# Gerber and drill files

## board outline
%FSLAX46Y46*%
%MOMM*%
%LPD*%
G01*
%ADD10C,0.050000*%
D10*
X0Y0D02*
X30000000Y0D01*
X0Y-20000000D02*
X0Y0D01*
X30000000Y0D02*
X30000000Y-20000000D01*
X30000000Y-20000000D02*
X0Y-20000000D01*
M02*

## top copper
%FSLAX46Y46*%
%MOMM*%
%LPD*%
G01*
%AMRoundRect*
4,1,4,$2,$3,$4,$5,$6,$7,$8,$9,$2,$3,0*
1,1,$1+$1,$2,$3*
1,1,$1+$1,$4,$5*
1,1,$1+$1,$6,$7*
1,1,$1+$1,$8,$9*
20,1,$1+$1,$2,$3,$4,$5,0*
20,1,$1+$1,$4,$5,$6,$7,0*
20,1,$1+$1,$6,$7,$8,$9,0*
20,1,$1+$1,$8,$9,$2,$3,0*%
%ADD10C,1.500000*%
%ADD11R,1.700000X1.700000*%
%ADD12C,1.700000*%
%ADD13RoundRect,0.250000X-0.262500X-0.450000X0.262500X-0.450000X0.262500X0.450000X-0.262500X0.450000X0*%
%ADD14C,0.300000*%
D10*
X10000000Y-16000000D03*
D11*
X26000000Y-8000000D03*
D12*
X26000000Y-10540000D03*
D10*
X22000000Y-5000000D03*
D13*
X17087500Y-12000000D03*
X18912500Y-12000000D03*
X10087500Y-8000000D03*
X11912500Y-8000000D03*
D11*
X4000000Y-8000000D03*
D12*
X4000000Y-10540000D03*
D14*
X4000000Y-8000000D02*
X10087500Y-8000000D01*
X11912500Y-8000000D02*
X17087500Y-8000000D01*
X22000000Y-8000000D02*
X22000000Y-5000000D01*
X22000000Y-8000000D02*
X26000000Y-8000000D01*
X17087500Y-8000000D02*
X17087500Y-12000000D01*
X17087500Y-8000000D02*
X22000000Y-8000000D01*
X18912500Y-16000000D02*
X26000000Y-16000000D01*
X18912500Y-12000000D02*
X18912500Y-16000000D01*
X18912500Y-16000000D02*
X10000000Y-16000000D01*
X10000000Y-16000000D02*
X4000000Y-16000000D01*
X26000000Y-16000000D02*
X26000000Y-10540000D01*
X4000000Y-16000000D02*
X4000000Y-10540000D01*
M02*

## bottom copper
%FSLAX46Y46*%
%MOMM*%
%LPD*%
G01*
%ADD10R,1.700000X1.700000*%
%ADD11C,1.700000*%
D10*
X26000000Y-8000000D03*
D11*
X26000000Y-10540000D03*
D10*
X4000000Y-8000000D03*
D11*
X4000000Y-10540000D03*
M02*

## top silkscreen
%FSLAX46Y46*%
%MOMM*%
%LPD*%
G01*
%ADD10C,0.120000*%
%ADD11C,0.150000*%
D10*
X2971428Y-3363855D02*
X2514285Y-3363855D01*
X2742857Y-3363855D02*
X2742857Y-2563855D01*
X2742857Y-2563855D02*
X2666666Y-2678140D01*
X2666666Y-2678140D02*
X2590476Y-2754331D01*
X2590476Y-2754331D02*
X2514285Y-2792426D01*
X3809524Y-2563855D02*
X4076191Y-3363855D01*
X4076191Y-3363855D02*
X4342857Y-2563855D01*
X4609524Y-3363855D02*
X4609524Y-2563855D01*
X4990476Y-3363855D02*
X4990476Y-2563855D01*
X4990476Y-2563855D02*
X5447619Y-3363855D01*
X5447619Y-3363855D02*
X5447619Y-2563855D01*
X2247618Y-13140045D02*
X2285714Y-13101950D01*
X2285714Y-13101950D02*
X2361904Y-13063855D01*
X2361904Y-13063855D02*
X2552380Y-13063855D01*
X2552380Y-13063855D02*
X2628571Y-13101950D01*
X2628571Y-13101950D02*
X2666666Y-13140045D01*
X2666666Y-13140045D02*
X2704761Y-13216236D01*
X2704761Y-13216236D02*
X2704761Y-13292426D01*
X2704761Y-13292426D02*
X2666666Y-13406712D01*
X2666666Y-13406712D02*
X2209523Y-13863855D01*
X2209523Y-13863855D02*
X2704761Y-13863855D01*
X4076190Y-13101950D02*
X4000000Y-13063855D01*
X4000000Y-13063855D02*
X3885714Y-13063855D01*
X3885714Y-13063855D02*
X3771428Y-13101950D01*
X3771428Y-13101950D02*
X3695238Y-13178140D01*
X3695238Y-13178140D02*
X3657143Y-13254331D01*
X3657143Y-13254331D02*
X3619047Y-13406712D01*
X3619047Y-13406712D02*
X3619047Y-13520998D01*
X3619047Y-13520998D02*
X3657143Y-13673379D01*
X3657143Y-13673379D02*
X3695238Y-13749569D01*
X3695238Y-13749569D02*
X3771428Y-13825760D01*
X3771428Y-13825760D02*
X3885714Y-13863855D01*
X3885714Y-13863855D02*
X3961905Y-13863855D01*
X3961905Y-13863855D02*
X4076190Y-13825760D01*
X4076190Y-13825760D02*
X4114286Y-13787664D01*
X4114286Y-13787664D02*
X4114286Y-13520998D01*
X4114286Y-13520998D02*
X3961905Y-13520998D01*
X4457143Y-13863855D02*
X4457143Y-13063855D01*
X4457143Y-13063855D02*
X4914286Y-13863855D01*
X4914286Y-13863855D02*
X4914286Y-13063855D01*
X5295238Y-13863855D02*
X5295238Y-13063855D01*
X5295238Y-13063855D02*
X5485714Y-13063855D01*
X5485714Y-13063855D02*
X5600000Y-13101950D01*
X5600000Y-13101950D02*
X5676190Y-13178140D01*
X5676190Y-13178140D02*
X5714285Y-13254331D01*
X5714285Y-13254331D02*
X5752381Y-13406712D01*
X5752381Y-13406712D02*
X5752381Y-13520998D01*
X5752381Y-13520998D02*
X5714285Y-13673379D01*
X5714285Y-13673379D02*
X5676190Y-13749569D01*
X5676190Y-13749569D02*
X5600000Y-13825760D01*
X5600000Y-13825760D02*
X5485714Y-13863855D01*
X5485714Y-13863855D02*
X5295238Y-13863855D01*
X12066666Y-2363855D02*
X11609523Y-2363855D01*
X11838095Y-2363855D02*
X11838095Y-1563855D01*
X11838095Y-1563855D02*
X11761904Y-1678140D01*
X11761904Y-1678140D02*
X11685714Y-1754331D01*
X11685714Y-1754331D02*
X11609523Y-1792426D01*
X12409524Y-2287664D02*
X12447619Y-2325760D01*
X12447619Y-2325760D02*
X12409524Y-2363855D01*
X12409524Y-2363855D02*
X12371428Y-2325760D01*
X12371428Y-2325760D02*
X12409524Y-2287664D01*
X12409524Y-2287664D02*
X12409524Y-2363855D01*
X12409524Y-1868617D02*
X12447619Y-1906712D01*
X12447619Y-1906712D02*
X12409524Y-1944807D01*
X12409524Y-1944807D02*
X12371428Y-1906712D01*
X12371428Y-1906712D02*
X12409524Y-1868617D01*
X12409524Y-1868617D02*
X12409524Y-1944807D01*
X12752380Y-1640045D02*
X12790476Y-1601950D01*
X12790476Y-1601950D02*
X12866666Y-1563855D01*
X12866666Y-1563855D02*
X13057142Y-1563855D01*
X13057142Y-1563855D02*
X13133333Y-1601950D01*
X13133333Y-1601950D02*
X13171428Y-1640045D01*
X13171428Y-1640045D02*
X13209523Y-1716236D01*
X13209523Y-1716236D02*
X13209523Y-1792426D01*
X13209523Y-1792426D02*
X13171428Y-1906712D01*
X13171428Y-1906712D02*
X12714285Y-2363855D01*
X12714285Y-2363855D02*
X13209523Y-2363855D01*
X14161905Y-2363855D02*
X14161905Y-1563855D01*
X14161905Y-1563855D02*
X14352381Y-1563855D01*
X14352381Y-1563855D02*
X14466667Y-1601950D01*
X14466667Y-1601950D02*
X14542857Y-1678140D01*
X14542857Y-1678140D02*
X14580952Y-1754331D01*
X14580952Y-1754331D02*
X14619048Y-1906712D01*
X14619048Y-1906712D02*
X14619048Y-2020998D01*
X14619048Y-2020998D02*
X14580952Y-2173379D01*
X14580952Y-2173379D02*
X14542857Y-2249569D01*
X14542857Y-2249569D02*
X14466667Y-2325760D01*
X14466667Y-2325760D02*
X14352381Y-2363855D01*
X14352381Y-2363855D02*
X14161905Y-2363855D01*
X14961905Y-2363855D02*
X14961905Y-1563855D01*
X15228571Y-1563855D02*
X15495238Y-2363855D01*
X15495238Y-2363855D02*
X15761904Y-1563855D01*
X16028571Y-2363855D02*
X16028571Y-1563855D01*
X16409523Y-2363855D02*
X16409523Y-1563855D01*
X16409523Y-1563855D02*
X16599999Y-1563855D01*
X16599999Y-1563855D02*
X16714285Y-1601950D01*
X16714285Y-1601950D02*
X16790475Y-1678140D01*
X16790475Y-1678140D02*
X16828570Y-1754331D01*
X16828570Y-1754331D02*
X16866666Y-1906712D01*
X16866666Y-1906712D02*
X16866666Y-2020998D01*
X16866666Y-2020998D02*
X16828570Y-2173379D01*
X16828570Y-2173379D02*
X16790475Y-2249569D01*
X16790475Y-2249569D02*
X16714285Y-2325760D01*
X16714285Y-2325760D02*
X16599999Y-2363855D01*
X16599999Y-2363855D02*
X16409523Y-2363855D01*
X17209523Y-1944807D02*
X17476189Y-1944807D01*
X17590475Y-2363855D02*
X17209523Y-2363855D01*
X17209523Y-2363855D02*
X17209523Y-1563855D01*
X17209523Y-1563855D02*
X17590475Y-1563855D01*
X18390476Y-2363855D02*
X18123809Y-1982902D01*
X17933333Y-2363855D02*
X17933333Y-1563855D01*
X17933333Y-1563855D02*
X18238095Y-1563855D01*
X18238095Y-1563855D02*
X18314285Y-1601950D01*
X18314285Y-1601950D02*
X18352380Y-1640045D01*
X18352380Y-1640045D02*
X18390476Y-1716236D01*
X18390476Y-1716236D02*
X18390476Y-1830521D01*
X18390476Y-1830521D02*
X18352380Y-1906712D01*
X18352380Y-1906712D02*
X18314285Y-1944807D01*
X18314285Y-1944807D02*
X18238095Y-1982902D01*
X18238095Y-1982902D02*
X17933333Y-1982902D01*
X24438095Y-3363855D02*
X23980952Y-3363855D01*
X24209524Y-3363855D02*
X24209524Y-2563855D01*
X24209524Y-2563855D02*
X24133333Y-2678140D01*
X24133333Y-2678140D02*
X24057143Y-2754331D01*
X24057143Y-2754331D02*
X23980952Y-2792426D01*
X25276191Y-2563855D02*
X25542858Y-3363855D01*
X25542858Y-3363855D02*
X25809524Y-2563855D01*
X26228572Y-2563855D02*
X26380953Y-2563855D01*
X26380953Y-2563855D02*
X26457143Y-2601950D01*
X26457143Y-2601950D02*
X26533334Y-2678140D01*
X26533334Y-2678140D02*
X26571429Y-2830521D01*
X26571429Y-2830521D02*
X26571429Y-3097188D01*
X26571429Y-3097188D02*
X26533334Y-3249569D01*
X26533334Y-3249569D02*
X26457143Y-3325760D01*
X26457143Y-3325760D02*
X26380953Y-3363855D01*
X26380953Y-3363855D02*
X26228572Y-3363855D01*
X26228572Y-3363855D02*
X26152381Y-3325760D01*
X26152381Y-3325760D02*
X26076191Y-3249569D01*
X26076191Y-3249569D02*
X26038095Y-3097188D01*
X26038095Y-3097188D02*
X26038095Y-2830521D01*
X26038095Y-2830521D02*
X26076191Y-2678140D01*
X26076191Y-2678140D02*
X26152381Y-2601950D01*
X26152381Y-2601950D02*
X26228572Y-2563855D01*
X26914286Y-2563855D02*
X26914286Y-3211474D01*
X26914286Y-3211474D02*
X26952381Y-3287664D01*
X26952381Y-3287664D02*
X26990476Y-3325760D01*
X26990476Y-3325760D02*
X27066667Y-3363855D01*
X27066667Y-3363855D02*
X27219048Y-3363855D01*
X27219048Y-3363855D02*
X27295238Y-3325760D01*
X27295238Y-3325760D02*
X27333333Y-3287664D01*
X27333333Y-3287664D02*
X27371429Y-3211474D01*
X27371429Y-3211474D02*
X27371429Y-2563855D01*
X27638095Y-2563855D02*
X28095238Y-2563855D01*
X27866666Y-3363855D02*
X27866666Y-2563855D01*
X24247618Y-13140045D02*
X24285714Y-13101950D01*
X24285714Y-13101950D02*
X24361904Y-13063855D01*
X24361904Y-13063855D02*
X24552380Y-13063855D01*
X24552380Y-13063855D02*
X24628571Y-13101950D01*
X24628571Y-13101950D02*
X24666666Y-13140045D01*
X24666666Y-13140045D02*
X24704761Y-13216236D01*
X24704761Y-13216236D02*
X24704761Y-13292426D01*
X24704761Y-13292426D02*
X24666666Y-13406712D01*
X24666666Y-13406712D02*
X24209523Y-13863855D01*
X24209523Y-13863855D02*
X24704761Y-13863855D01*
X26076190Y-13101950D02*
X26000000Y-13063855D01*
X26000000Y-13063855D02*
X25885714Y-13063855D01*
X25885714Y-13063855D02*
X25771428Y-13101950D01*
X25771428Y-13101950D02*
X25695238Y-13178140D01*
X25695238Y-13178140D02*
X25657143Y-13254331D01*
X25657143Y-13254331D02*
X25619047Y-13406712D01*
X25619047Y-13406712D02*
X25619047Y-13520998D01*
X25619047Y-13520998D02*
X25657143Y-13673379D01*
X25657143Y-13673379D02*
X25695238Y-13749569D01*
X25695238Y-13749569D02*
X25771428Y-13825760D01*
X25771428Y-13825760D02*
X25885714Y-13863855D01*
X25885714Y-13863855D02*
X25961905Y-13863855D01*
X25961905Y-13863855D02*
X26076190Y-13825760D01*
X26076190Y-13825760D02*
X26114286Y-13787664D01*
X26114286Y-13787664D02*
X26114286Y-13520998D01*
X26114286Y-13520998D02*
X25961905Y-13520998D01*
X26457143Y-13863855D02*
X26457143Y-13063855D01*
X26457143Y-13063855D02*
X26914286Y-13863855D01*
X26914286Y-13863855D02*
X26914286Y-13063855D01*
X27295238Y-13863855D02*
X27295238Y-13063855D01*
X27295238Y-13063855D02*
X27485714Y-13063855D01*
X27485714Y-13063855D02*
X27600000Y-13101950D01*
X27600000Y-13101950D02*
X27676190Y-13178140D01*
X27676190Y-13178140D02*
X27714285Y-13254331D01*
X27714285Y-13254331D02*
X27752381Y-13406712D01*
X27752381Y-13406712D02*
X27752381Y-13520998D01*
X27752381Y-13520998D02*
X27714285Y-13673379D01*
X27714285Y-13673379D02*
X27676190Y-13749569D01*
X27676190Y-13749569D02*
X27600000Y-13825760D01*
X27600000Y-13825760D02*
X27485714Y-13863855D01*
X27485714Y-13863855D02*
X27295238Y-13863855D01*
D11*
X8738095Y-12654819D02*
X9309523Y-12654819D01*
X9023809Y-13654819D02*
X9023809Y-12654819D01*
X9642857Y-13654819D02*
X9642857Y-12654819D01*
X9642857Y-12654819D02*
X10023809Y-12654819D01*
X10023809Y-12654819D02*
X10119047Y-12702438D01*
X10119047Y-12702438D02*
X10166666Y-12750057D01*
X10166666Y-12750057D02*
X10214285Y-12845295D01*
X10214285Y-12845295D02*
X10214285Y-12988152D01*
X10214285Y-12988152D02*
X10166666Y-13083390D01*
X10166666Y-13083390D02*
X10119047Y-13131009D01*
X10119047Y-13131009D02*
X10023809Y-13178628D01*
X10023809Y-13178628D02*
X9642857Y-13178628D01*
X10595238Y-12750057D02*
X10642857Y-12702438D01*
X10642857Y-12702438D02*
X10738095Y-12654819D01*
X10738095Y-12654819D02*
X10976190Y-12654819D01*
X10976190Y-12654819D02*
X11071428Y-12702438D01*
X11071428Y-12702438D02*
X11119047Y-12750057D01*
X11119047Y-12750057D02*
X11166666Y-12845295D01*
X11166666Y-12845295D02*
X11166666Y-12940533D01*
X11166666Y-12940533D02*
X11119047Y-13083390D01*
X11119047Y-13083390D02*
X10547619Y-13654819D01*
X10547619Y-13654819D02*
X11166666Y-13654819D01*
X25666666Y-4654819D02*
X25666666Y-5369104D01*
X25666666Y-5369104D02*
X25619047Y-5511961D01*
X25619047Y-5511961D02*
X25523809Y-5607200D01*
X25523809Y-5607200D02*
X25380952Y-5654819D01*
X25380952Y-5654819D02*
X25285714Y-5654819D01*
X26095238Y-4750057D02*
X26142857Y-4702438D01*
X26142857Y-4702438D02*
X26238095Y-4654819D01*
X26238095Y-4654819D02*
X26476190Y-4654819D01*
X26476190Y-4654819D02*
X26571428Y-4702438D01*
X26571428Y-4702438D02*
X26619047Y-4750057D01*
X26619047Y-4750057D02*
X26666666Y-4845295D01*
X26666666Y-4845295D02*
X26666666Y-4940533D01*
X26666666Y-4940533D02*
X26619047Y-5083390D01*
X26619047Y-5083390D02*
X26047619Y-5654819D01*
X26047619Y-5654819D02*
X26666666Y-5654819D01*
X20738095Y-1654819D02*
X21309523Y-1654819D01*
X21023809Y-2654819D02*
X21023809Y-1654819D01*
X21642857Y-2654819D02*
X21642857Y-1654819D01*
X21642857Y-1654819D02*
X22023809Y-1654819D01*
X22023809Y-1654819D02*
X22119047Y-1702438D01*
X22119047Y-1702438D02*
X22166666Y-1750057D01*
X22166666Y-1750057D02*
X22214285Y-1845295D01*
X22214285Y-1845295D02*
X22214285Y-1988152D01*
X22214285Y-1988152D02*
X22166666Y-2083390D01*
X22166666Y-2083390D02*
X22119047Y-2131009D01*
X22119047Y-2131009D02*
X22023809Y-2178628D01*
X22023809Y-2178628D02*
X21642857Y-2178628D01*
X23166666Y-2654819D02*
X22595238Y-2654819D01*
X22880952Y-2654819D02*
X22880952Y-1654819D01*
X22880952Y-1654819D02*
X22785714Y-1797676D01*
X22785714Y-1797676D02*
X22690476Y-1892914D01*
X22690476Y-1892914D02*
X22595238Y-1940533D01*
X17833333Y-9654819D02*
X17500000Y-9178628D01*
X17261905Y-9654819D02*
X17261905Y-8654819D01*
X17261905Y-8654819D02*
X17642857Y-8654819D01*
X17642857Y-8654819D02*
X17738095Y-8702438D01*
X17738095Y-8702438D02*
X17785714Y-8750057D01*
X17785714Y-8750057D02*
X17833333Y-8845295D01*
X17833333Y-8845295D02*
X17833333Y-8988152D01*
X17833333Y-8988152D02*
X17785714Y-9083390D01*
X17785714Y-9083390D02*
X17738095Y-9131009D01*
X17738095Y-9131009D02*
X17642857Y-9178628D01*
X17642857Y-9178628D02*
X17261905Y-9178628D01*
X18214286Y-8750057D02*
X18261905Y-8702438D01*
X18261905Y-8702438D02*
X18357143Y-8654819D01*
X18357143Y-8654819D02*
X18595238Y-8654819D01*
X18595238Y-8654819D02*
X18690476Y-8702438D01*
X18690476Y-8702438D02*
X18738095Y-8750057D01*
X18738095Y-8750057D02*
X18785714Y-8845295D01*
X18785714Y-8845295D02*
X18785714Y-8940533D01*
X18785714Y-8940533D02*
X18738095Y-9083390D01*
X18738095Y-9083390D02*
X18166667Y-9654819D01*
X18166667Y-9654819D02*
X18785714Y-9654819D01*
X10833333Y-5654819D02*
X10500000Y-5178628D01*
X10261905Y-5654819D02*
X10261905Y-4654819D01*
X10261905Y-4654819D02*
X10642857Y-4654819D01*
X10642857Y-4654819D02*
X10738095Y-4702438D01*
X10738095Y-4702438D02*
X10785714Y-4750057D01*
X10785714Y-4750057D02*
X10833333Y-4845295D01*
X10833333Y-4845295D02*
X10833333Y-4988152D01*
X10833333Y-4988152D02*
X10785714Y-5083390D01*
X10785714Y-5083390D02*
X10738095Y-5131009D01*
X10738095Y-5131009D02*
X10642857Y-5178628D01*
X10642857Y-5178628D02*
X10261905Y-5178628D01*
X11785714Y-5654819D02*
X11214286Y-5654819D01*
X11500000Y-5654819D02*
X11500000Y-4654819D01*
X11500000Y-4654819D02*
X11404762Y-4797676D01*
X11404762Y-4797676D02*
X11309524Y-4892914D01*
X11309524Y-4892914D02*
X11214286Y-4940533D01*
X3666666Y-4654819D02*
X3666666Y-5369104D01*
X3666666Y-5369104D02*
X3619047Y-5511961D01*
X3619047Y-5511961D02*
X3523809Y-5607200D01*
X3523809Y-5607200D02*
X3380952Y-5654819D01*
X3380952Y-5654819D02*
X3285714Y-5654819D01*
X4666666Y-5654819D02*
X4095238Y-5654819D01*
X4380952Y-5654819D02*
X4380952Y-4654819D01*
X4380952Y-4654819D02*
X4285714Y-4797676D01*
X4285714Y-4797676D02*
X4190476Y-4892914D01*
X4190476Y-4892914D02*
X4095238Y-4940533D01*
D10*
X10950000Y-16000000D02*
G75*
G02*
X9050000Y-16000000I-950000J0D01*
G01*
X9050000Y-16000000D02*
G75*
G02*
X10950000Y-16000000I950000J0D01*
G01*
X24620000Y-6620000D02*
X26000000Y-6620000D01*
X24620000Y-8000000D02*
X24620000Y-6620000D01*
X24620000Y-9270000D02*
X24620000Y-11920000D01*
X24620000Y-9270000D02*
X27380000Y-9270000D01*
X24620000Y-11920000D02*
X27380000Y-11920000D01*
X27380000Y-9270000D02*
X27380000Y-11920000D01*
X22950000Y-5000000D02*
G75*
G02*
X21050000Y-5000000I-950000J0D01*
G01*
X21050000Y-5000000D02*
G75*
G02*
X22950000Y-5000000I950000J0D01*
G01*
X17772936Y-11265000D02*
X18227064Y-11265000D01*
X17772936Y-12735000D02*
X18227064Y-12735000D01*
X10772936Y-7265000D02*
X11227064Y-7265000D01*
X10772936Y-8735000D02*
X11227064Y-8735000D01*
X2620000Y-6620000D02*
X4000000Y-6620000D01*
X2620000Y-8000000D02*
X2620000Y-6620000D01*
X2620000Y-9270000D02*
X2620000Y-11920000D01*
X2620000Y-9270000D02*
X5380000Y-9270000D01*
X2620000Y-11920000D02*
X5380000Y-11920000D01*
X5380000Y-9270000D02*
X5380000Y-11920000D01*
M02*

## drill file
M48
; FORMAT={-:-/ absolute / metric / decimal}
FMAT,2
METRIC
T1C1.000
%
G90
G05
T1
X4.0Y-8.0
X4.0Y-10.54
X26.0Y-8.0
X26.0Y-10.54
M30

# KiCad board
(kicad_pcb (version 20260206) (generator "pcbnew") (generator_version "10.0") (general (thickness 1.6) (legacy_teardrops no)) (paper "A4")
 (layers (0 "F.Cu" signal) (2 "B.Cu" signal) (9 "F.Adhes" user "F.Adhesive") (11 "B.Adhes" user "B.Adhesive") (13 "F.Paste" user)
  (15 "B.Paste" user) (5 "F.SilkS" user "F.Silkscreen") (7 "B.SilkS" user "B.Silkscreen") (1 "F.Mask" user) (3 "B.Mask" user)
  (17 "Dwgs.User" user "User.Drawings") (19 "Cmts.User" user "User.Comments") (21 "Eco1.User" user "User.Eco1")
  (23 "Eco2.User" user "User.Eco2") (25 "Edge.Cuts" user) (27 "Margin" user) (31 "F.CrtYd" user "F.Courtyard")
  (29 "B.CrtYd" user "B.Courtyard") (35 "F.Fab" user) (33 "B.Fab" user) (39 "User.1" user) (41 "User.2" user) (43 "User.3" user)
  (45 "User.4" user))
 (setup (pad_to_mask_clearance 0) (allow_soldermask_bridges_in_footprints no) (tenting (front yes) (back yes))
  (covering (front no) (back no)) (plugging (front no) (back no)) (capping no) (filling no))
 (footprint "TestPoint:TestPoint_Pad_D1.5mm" (layer "F.Cu") (at 10 16)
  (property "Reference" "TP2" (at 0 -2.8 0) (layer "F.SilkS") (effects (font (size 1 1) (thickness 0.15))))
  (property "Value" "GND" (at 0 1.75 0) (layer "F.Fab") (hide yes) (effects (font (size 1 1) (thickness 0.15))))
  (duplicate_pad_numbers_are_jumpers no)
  (fp_circle (center 0 0) (end 0 0.95) (stroke (width 0.12) (type solid)) (fill no) (layer "F.SilkS"))
  (pad "1" smd circle (at 0 0) (size 1.5 1.5) (layers "F.Cu" "F.Mask") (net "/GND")))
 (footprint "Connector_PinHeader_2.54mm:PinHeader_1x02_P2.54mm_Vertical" (layer "F.Cu") (at 26 8)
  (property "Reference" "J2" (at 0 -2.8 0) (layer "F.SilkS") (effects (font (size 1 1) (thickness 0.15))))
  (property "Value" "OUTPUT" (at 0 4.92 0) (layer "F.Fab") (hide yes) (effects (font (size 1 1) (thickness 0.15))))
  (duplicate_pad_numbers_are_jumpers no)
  (fp_line (start -1.38 -1.38) (end 0 -1.38) (stroke (width 0.12) (type solid)) (layer "F.SilkS"))
  (fp_line (start -1.38 0) (end -1.38 -1.38) (stroke (width 0.12) (type solid)) (layer "F.SilkS"))
  (fp_line (start -1.38 1.27) (end -1.38 3.92) (stroke (width 0.12) (type solid)) (layer "F.SilkS"))
  (fp_line (start -1.38 1.27) (end 1.38 1.27) (stroke (width 0.12) (type solid)) (layer "F.SilkS"))
  (fp_line (start -1.38 3.92) (end 1.38 3.92) (stroke (width 0.12) (type solid)) (layer "F.SilkS"))
  (fp_line (start 1.38 1.27) (end 1.38 3.92) (stroke (width 0.12) (type solid)) (layer "F.SilkS"))
  (pad "1" thru_hole rect (at 0 0) (size 1.7 1.7) (drill 1) (layers "*.Cu" "*.Mask") (remove_unused_layers no) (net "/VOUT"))
  (pad "2" thru_hole circle (at 0 2.54) (size 1.7 1.7) (drill 1) (layers "*.Cu" "*.Mask") (remove_unused_layers no) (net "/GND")))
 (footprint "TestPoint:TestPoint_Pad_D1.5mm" (layer "F.Cu") (at 22 5)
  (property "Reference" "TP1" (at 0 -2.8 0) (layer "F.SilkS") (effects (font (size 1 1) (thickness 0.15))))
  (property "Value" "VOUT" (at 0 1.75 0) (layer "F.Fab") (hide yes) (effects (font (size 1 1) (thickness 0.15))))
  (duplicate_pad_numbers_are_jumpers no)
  (fp_circle (center 0 0) (end 0 0.95) (stroke (width 0.12) (type solid)) (fill no) (layer "F.SilkS"))
  (pad "1" smd circle (at 0 0) (size 1.5 1.5) (layers "F.Cu" "F.Mask") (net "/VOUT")))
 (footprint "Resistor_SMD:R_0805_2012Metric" (layer "F.Cu") (at 18 12)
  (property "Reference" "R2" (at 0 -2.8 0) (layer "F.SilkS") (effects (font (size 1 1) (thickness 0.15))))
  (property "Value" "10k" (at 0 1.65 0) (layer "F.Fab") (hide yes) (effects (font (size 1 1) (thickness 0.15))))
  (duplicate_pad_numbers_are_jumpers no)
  (fp_line (start -0.227064 -0.735) (end 0.227064 -0.735) (stroke (width 0.12) (type solid)) (layer "F.SilkS"))
  (fp_line (start -0.227064 0.735) (end 0.227064 0.735) (stroke (width 0.12) (type solid)) (layer "F.SilkS"))
  (pad "1" smd roundrect (at -0.9125 0) (size 1.025 1.4) (layers "F.Cu" "F.Mask" "F.Paste") (roundrect_rratio 0.243902) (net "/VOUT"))
  (pad "2" smd roundrect (at 0.9125 0) (size 1.025 1.4) (layers "F.Cu" "F.Mask" "F.Paste") (roundrect_rratio 0.243902) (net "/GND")))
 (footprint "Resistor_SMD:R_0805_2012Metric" (layer "F.Cu") (at 11 8)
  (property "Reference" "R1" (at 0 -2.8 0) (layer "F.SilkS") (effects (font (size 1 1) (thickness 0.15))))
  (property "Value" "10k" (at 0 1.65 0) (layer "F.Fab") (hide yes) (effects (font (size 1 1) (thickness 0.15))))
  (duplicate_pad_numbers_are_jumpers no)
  (fp_line (start -0.227064 -0.735) (end 0.227064 -0.735) (stroke (width 0.12) (type solid)) (layer "F.SilkS"))
  (fp_line (start -0.227064 0.735) (end 0.227064 0.735) (stroke (width 0.12) (type solid)) (layer "F.SilkS"))
  (pad "1" smd roundrect (at -0.9125 0) (size 1.025 1.4) (layers "F.Cu" "F.Mask" "F.Paste") (roundrect_rratio 0.243902) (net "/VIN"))
  (pad "2" smd roundrect (at 0.9125 0) (size 1.025 1.4) (layers "F.Cu" "F.Mask" "F.Paste") (roundrect_rratio 0.243902) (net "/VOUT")))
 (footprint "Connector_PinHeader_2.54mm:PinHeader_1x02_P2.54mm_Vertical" (layer "F.Cu") (at 4 8)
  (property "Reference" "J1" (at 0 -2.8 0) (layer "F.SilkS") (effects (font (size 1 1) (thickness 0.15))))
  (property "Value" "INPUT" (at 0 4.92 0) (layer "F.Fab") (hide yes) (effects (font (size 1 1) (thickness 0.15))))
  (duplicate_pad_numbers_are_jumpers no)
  (fp_line (start -1.38 -1.38) (end 0 -1.38) (stroke (width 0.12) (type solid)) (layer "F.SilkS"))
  (fp_line (start -1.38 0) (end -1.38 -1.38) (stroke (width 0.12) (type solid)) (layer "F.SilkS"))
  (fp_line (start -1.38 1.27) (end -1.38 3.92) (stroke (width 0.12) (type solid)) (layer "F.SilkS"))
  (fp_line (start -1.38 1.27) (end 1.38 1.27) (stroke (width 0.12) (type solid)) (layer "F.SilkS"))
  (fp_line (start -1.38 3.92) (end 1.38 3.92) (stroke (width 0.12) (type solid)) (layer "F.SilkS"))
  (fp_line (start 1.38 1.27) (end 1.38 3.92) (stroke (width 0.12) (type solid)) (layer "F.SilkS"))
  (pad "1" thru_hole rect (at 0 0) (size 1.7 1.7) (drill 1) (layers "*.Cu" "*.Mask") (remove_unused_layers no) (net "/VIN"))
  (pad "2" thru_hole circle (at 0 2.54) (size 1.7 1.7) (drill 1) (layers "*.Cu" "*.Mask") (remove_unused_layers no) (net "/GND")))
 (gr_line (start 0 0) (end 30 0) (stroke (width 0.05) (type default)) (layer "Edge.Cuts"))
 (gr_line (start 0 20) (end 0 0) (stroke (width 0.05) (type default)) (layer "Edge.Cuts"))
 (gr_line (start 30 0) (end 30 20) (stroke (width 0.05) (type default)) (layer "Edge.Cuts"))
 (gr_line (start 30 20) (end 0 20) (stroke (width 0.05) (type default)) (layer "Edge.Cuts"))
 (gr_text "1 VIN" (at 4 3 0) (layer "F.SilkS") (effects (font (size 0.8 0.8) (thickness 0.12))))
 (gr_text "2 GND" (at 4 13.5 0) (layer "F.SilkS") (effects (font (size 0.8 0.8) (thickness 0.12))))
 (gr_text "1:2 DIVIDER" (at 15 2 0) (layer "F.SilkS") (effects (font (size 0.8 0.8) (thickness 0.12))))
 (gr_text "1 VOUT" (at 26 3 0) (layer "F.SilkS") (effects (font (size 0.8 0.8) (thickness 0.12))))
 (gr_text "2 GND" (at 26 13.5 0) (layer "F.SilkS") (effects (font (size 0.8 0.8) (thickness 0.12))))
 (segment (start 4 8) (end 10.0875 8) (width 0.3) (layer "F.Cu") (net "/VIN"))
 (segment (start 11.9125 8) (end 17.0875 8) (width 0.3) (layer "F.Cu") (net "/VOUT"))
 (segment (start 22 8) (end 22 5) (width 0.3) (layer "F.Cu") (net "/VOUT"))
 (segment (start 22 8) (end 26 8) (width 0.3) (layer "F.Cu") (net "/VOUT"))
 (segment (start 17.0875 8) (end 17.0875 12) (width 0.3) (layer "F.Cu") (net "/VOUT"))
 (segment (start 17.0875 8) (end 22 8) (width 0.3) (layer "F.Cu") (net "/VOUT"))
 (segment (start 18.9125 16) (end 26 16) (width 0.3) (layer "F.Cu") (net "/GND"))
 (segment (start 18.9125 12) (end 18.9125 16) (width 0.3) (layer "F.Cu") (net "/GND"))
 (segment (start 18.9125 16) (end 10 16) (width 0.3) (layer "F.Cu") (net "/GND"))
 (segment (start 10 16) (end 4 16) (width 0.3) (layer "F.Cu") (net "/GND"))
 (segment (start 26 16) (end 26 10.54) (width 0.3) (layer "F.Cu") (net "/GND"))
 (segment (start 4 16) (end 4 10.54) (width 0.3) (layer "F.Cu") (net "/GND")))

